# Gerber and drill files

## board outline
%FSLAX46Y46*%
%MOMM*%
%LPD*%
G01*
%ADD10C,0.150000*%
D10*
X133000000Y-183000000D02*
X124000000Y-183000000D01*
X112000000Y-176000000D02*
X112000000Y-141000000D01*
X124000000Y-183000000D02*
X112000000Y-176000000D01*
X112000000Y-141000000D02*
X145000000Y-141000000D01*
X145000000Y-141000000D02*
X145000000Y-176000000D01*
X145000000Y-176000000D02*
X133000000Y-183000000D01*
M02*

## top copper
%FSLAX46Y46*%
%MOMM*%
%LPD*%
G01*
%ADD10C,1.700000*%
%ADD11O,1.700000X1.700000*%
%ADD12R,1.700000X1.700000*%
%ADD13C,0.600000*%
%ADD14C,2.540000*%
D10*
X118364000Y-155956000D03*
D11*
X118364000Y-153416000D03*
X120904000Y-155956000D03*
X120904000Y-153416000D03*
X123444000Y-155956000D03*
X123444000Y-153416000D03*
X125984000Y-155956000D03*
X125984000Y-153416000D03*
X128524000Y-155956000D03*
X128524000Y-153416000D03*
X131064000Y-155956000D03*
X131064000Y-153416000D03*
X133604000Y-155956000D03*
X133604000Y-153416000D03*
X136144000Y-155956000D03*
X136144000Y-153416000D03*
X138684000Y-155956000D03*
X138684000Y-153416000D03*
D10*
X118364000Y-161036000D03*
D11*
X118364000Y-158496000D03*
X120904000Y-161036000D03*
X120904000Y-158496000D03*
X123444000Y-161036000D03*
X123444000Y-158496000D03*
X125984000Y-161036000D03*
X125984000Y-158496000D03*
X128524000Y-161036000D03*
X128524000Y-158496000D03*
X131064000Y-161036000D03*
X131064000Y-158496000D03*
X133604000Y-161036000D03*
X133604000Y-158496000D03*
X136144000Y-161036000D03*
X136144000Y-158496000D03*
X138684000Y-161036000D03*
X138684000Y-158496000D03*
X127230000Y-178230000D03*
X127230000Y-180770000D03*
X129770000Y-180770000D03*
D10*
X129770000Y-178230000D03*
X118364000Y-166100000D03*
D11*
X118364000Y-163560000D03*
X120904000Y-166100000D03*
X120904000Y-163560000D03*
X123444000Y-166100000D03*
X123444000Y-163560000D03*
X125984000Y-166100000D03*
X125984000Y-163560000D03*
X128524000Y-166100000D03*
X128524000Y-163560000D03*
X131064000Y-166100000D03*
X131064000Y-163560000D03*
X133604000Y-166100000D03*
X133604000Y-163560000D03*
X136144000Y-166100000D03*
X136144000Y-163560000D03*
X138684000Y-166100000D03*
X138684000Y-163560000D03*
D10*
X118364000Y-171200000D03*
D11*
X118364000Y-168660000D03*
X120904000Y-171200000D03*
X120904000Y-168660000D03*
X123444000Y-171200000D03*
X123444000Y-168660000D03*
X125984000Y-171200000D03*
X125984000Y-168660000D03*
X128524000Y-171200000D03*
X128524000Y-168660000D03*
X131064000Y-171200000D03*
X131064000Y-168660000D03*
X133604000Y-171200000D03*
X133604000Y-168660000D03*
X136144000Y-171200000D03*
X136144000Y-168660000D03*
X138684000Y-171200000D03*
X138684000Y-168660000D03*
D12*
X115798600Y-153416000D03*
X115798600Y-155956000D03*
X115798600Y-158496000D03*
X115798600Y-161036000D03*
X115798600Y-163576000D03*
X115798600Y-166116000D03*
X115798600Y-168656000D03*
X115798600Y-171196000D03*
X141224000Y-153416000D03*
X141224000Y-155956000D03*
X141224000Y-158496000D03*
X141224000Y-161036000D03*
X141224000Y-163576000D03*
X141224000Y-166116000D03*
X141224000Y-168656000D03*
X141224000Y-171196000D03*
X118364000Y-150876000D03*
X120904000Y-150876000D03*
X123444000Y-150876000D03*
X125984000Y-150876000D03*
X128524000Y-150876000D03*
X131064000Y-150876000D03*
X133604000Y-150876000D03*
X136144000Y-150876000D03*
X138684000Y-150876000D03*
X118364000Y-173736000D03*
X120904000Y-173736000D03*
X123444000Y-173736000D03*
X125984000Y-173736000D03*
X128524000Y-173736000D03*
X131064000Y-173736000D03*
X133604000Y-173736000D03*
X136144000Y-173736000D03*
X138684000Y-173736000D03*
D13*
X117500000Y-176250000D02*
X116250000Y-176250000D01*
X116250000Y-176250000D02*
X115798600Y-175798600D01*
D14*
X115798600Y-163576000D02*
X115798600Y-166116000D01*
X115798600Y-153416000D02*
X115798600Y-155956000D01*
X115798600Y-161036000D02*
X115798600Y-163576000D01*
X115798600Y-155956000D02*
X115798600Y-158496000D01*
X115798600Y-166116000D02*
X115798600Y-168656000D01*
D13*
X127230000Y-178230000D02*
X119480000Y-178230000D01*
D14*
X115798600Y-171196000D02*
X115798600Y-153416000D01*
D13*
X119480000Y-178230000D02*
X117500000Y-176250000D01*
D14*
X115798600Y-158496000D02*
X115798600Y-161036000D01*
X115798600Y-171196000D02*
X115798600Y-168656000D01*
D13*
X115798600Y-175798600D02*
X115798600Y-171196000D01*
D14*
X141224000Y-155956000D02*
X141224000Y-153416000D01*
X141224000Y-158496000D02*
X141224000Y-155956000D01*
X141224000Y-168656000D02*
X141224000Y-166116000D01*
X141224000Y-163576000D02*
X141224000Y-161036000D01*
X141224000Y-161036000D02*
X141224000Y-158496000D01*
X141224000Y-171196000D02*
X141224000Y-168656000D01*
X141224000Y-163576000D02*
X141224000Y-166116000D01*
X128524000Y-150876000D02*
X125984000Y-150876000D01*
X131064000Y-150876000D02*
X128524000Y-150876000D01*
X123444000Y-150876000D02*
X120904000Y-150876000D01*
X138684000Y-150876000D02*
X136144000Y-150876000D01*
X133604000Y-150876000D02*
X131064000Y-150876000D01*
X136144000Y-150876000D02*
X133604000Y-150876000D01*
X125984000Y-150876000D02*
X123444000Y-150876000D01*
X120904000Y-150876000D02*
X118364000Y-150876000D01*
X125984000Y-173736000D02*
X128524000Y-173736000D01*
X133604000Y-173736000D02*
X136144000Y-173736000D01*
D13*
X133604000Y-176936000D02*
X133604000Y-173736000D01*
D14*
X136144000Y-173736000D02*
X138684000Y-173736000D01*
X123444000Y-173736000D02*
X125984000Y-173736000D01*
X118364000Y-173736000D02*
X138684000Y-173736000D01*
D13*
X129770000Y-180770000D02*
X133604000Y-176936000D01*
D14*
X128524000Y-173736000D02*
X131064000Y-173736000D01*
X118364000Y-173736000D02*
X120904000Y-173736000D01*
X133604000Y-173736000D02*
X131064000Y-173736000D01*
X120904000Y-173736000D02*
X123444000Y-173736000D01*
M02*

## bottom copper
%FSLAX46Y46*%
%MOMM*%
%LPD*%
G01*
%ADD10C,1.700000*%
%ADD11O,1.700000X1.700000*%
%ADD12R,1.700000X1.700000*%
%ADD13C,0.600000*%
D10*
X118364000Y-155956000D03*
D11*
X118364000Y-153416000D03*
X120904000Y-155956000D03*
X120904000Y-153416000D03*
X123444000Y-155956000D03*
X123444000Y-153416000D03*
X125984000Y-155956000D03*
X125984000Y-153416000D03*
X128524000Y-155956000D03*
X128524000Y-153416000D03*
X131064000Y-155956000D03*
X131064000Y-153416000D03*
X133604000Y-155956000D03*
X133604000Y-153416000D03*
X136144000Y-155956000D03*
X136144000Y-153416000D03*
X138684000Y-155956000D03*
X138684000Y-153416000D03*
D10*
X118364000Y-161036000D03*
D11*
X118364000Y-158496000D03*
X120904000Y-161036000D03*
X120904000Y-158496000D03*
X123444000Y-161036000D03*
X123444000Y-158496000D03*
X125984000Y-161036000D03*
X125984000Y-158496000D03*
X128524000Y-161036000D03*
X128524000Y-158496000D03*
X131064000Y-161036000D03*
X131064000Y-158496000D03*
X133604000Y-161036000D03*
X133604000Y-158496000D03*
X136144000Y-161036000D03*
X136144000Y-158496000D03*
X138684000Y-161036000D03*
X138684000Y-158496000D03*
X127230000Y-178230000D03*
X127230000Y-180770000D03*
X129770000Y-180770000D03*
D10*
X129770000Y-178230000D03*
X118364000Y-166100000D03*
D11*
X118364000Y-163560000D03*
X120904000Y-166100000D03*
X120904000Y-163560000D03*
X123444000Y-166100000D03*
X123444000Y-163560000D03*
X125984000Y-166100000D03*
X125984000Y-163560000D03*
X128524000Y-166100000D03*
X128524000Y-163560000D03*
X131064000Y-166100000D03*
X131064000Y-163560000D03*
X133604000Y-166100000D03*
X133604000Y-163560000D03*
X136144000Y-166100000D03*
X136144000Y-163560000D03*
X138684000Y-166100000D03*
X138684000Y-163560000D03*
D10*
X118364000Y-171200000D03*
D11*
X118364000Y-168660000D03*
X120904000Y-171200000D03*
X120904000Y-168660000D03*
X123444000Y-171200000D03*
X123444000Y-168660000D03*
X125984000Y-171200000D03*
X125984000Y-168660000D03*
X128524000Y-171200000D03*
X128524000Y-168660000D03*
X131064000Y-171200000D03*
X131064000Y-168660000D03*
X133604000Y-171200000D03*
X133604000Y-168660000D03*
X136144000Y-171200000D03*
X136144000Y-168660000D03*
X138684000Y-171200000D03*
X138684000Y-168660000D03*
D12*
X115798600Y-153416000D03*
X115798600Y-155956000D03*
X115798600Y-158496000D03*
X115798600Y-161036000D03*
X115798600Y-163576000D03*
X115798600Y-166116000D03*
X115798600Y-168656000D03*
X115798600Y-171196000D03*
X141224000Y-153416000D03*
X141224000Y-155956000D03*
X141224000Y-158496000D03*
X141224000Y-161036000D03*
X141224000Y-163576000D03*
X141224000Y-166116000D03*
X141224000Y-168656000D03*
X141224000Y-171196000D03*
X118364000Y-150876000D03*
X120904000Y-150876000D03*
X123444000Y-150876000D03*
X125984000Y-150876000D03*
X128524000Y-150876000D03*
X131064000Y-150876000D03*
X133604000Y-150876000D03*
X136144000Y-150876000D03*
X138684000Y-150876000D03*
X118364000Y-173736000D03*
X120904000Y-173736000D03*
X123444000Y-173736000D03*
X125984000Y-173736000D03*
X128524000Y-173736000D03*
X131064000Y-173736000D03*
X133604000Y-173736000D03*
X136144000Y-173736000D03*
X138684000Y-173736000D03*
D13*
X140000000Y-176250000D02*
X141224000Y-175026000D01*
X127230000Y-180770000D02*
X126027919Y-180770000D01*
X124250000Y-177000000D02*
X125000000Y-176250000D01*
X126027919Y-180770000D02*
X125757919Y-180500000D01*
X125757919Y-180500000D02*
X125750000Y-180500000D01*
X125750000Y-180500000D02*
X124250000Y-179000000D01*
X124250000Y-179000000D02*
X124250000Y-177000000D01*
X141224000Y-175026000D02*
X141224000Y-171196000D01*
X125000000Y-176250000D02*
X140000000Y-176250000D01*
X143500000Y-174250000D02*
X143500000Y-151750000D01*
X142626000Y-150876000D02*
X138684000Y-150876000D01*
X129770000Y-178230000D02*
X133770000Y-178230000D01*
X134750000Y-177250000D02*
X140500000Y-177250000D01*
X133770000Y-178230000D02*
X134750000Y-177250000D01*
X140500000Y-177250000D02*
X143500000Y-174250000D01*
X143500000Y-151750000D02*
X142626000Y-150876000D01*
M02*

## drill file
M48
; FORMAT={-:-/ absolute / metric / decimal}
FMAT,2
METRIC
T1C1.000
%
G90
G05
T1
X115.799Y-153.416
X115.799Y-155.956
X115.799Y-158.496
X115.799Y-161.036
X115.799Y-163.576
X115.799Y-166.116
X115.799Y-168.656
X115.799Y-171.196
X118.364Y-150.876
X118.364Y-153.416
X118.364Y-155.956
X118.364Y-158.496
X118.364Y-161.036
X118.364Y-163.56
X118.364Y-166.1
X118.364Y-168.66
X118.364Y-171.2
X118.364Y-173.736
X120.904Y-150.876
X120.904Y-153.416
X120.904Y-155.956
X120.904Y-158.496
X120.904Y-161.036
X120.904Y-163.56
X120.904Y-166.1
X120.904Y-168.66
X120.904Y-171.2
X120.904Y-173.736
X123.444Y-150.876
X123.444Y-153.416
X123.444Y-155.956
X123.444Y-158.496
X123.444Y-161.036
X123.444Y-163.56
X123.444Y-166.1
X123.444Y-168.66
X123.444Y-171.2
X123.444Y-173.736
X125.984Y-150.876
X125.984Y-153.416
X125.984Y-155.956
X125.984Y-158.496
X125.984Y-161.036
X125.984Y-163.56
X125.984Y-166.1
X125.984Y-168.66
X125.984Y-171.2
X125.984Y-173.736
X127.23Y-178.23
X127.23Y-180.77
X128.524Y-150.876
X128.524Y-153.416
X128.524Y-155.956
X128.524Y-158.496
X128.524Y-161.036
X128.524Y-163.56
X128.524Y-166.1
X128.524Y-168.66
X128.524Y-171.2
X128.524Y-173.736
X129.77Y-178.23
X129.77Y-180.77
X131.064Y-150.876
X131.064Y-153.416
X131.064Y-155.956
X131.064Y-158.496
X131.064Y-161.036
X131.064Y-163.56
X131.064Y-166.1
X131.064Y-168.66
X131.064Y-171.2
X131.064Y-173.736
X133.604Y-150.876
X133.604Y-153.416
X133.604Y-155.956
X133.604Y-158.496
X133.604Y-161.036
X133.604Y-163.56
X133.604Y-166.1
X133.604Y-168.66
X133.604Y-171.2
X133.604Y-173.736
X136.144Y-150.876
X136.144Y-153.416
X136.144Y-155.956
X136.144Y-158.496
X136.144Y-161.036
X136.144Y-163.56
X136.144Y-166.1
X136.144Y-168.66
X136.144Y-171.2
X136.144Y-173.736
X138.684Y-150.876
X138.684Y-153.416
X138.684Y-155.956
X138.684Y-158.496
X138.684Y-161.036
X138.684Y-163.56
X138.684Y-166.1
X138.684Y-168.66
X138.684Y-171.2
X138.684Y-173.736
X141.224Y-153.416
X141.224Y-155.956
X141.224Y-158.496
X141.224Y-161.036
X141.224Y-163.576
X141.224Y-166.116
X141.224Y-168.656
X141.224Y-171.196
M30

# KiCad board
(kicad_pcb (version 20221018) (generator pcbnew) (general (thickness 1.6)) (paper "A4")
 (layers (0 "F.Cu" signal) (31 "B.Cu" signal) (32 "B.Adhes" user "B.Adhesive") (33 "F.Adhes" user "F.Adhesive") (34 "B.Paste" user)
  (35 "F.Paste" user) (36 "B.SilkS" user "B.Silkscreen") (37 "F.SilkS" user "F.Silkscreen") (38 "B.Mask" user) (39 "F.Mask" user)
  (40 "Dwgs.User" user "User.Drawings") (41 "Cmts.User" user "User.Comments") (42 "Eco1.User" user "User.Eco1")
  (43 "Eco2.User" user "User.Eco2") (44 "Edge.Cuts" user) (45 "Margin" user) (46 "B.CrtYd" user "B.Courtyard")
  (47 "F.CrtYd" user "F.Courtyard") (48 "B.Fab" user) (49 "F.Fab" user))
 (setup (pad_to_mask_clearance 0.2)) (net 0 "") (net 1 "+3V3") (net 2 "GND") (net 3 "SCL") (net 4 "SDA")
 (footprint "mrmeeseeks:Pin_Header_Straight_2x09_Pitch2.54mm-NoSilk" (layer "F.Cu") (at 118.364 155.956 90)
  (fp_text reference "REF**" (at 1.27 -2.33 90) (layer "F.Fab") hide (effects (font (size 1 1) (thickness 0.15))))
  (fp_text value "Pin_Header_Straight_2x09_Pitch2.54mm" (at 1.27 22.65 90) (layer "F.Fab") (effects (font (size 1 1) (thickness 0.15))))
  (pad "1" thru_hole circle (at 0 0 90) (size 1.7 1.7) (drill 1) (layers "*.Cu" "*.Mask"))
  (pad "2" thru_hole oval (at 2.54 0 90) (size 1.7 1.7) (drill 1) (layers "*.Cu" "*.Mask"))
  (pad "3" thru_hole oval (at 0 2.54 90) (size 1.7 1.7) (drill 1) (layers "*.Cu" "*.Mask"))
  (pad "4" thru_hole oval (at 2.54 2.54 90) (size 1.7 1.7) (drill 1) (layers "*.Cu" "*.Mask"))
  (pad "5" thru_hole oval (at 0 5.08 90) (size 1.7 1.7) (drill 1) (layers "*.Cu" "*.Mask"))
  (pad "6" thru_hole oval (at 2.54 5.08 90) (size 1.7 1.7) (drill 1) (layers "*.Cu" "*.Mask"))
  (pad "7" thru_hole oval (at 0 7.62 90) (size 1.7 1.7) (drill 1) (layers "*.Cu" "*.Mask"))
  (pad "8" thru_hole oval (at 2.54 7.62 90) (size 1.7 1.7) (drill 1) (layers "*.Cu" "*.Mask"))
  (pad "9" thru_hole oval (at 0 10.16 90) (size 1.7 1.7) (drill 1) (layers "*.Cu" "*.Mask"))
  (pad "10" thru_hole oval (at 2.54 10.16 90) (size 1.7 1.7) (drill 1) (layers "*.Cu" "*.Mask"))
  (pad "11" thru_hole oval (at 0 12.7 90) (size 1.7 1.7) (drill 1) (layers "*.Cu" "*.Mask"))
  (pad "12" thru_hole oval (at 2.54 12.7 90) (size 1.7 1.7) (drill 1) (layers "*.Cu" "*.Mask"))
  (pad "13" thru_hole oval (at 0 15.24 90) (size 1.7 1.7) (drill 1) (layers "*.Cu" "*.Mask"))
  (pad "14" thru_hole oval (at 2.54 15.24 90) (size 1.7 1.7) (drill 1) (layers "*.Cu" "*.Mask"))
  (pad "15" thru_hole oval (at 0 17.78 90) (size 1.7 1.7) (drill 1) (layers "*.Cu" "*.Mask"))
  (pad "16" thru_hole oval (at 2.54 17.78 90) (size 1.7 1.7) (drill 1) (layers "*.Cu" "*.Mask"))
  (pad "17" thru_hole oval (at 0 20.32 90) (size 1.7 1.7) (drill 1) (layers "*.Cu" "*.Mask"))
  (pad "18" thru_hole oval (at 2.54 20.32 90) (size 1.7 1.7) (drill 1) (layers "*.Cu" "*.Mask")))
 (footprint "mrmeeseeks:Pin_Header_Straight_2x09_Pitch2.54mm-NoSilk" (layer "F.Cu") (at 118.364 161.036 90)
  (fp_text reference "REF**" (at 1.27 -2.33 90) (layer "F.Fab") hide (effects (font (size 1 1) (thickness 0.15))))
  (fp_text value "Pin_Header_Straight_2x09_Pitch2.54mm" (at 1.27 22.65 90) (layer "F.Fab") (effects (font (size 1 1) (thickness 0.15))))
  (pad "1" thru_hole circle (at 0 0 90) (size 1.7 1.7) (drill 1) (layers "*.Cu" "*.Mask"))
  (pad "2" thru_hole oval (at 2.54 0 90) (size 1.7 1.7) (drill 1) (layers "*.Cu" "*.Mask"))
  (pad "3" thru_hole oval (at 0 2.54 90) (size 1.7 1.7) (drill 1) (layers "*.Cu" "*.Mask"))
  (pad "4" thru_hole oval (at 2.54 2.54 90) (size 1.7 1.7) (drill 1) (layers "*.Cu" "*.Mask"))
  (pad "5" thru_hole oval (at 0 5.08 90) (size 1.7 1.7) (drill 1) (layers "*.Cu" "*.Mask"))
  (pad "6" thru_hole oval (at 2.54 5.08 90) (size 1.7 1.7) (drill 1) (layers "*.Cu" "*.Mask"))
  (pad "7" thru_hole oval (at 0 7.62 90) (size 1.7 1.7) (drill 1) (layers "*.Cu" "*.Mask"))
  (pad "8" thru_hole oval (at 2.54 7.62 90) (size 1.7 1.7) (drill 1) (layers "*.Cu" "*.Mask"))
  (pad "9" thru_hole oval (at 0 10.16 90) (size 1.7 1.7) (drill 1) (layers "*.Cu" "*.Mask"))
  (pad "10" thru_hole oval (at 2.54 10.16 90) (size 1.7 1.7) (drill 1) (layers "*.Cu" "*.Mask"))
  (pad "11" thru_hole oval (at 0 12.7 90) (size 1.7 1.7) (drill 1) (layers "*.Cu" "*.Mask"))
  (pad "12" thru_hole oval (at 2.54 12.7 90) (size 1.7 1.7) (drill 1) (layers "*.Cu" "*.Mask"))
  (pad "13" thru_hole oval (at 0 15.24 90) (size 1.7 1.7) (drill 1) (layers "*.Cu" "*.Mask"))
  (pad "14" thru_hole oval (at 2.54 15.24 90) (size 1.7 1.7) (drill 1) (layers "*.Cu" "*.Mask"))
  (pad "15" thru_hole oval (at 0 17.78 90) (size 1.7 1.7) (drill 1) (layers "*.Cu" "*.Mask"))
  (pad "16" thru_hole oval (at 2.54 17.78 90) (size 1.7 1.7) (drill 1) (layers "*.Cu" "*.Mask"))
  (pad "17" thru_hole oval (at 0 20.32 90) (size 1.7 1.7) (drill 1) (layers "*.Cu" "*.Mask"))
  (pad "18" thru_hole oval (at 2.54 20.32 90) (size 1.7 1.7) (drill 1) (layers "*.Cu" "*.Mask")))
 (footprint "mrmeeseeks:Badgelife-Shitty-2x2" (layer "F.Cu") (at 128.5 179.5)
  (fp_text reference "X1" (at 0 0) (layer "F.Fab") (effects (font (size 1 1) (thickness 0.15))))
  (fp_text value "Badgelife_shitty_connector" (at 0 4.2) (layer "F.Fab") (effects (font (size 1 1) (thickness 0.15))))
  (pad "1" thru_hole oval (at -1.27 -1.27) (size 1.7 1.7) (drill 1) (layers "*.Cu" "*.Mask") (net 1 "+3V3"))
  (pad "2" thru_hole oval (at -1.27 1.27) (size 1.7 1.7) (drill 1) (layers "*.Cu" "*.Mask") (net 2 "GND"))
  (pad "3" thru_hole oval (at 1.27 1.27) (size 1.7 1.7) (drill 1) (layers "*.Cu" "*.Mask") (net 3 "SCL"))
  (pad "4" thru_hole circle (at 1.27 -1.27) (size 1.7 1.7) (drill 1) (layers "*.Cu" "*.Mask") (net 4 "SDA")))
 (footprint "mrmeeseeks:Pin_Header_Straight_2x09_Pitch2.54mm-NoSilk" (layer "F.Cu") (at 118.364 166.1 90)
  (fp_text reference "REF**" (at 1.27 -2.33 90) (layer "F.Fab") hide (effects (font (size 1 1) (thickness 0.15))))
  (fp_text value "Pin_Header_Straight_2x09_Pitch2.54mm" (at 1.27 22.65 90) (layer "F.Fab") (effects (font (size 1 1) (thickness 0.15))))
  (pad "1" thru_hole circle (at 0 0 90) (size 1.7 1.7) (drill 1) (layers "*.Cu" "*.Mask"))
  (pad "2" thru_hole oval (at 2.54 0 90) (size 1.7 1.7) (drill 1) (layers "*.Cu" "*.Mask"))
  (pad "3" thru_hole oval (at 0 2.54 90) (size 1.7 1.7) (drill 1) (layers "*.Cu" "*.Mask"))
  (pad "4" thru_hole oval (at 2.54 2.54 90) (size 1.7 1.7) (drill 1) (layers "*.Cu" "*.Mask"))
  (pad "5" thru_hole oval (at 0 5.08 90) (size 1.7 1.7) (drill 1) (layers "*.Cu" "*.Mask"))
  (pad "6" thru_hole oval (at 2.54 5.08 90) (size 1.7 1.7) (drill 1) (layers "*.Cu" "*.Mask"))
  (pad "7" thru_hole oval (at 0 7.62 90) (size 1.7 1.7) (drill 1) (layers "*.Cu" "*.Mask"))
  (pad "8" thru_hole oval (at 2.54 7.62 90) (size 1.7 1.7) (drill 1) (layers "*.Cu" "*.Mask"))
  (pad "9" thru_hole oval (at 0 10.16 90) (size 1.7 1.7) (drill 1) (layers "*.Cu" "*.Mask"))
  (pad "10" thru_hole oval (at 2.54 10.16 90) (size 1.7 1.7) (drill 1) (layers "*.Cu" "*.Mask"))
  (pad "11" thru_hole oval (at 0 12.7 90) (size 1.7 1.7) (drill 1) (layers "*.Cu" "*.Mask"))
  (pad "12" thru_hole oval (at 2.54 12.7 90) (size 1.7 1.7) (drill 1) (layers "*.Cu" "*.Mask"))
  (pad "13" thru_hole oval (at 0 15.24 90) (size 1.7 1.7) (drill 1) (layers "*.Cu" "*.Mask"))
  (pad "14" thru_hole oval (at 2.54 15.24 90) (size 1.7 1.7) (drill 1) (layers "*.Cu" "*.Mask"))
  (pad "15" thru_hole oval (at 0 17.78 90) (size 1.7 1.7) (drill 1) (layers "*.Cu" "*.Mask"))
  (pad "16" thru_hole oval (at 2.54 17.78 90) (size 1.7 1.7) (drill 1) (layers "*.Cu" "*.Mask"))
  (pad "17" thru_hole oval (at 0 20.32 90) (size 1.7 1.7) (drill 1) (layers "*.Cu" "*.Mask"))
  (pad "18" thru_hole oval (at 2.54 20.32 90) (size 1.7 1.7) (drill 1) (layers "*.Cu" "*.Mask")))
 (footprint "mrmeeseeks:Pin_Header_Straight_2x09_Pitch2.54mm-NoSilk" (layer "F.Cu") (at 118.364 171.2 90)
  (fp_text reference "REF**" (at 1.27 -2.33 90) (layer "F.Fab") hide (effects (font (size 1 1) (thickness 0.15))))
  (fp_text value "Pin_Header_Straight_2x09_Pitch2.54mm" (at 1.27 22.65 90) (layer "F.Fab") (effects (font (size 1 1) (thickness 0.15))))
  (pad "1" thru_hole circle (at 0 0 90) (size 1.7 1.7) (drill 1) (layers "*.Cu" "*.Mask"))
  (pad "2" thru_hole oval (at 2.54 0 90) (size 1.7 1.7) (drill 1) (layers "*.Cu" "*.Mask"))
  (pad "3" thru_hole oval (at 0 2.54 90) (size 1.7 1.7) (drill 1) (layers "*.Cu" "*.Mask"))
  (pad "4" thru_hole oval (at 2.54 2.54 90) (size 1.7 1.7) (drill 1) (layers "*.Cu" "*.Mask"))
  (pad "5" thru_hole oval (at 0 5.08 90) (size 1.7 1.7) (drill 1) (layers "*.Cu" "*.Mask"))
  (pad "6" thru_hole oval (at 2.54 5.08 90) (size 1.7 1.7) (drill 1) (layers "*.Cu" "*.Mask"))
  (pad "7" thru_hole oval (at 0 7.62 90) (size 1.7 1.7) (drill 1) (layers "*.Cu" "*.Mask"))
  (pad "8" thru_hole oval (at 2.54 7.62 90) (size 1.7 1.7) (drill 1) (layers "*.Cu" "*.Mask"))
  (pad "9" thru_hole oval (at 0 10.16 90) (size 1.7 1.7) (drill 1) (layers "*.Cu" "*.Mask"))
  (pad "10" thru_hole oval (at 2.54 10.16 90) (size 1.7 1.7) (drill 1) (layers "*.Cu" "*.Mask"))
  (pad "11" thru_hole oval (at 0 12.7 90) (size 1.7 1.7) (drill 1) (layers "*.Cu" "*.Mask"))
  (pad "12" thru_hole oval (at 2.54 12.7 90) (size 1.7 1.7) (drill 1) (layers "*.Cu" "*.Mask"))
  (pad "13" thru_hole oval (at 0 15.24 90) (size 1.7 1.7) (drill 1) (layers "*.Cu" "*.Mask"))
  (pad "14" thru_hole oval (at 2.54 15.24 90) (size 1.7 1.7) (drill 1) (layers "*.Cu" "*.Mask"))
  (pad "15" thru_hole oval (at 0 17.78 90) (size 1.7 1.7) (drill 1) (layers "*.Cu" "*.Mask"))
  (pad "16" thru_hole oval (at 2.54 17.78 90) (size 1.7 1.7) (drill 1) (layers "*.Cu" "*.Mask"))
  (pad "17" thru_hole oval (at 0 20.32 90) (size 1.7 1.7) (drill 1) (layers "*.Cu" "*.Mask"))
  (pad "18" thru_hole oval (at 2.54 20.32 90) (size 1.7 1.7) (drill 1) (layers "*.Cu" "*.Mask")))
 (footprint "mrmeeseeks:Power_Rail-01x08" (layer "F.Cu") (at 115.7986 153.416)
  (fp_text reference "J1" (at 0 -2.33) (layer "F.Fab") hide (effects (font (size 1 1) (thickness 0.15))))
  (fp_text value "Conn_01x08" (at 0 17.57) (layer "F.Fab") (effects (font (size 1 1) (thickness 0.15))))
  (pad "1" thru_hole rect (at 0 0) (size 1.7 1.7) (drill 1) (layers "*.Cu" "*.Mask") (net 1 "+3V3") (solder_mask_margin 0.1))
  (pad "2" thru_hole rect (at 0 2.54) (size 1.7 1.7) (drill 1) (layers "*.Cu" "*.Mask") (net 1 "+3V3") (solder_mask_margin 0.1))
  (pad "3" thru_hole rect (at 0 5.08) (size 1.7 1.7) (drill 1) (layers "*.Cu" "*.Mask") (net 1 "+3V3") (solder_mask_margin 0.1))
  (pad "4" thru_hole rect (at 0 7.62) (size 1.7 1.7) (drill 1) (layers "*.Cu" "*.Mask") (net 1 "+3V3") (solder_mask_margin 0.1))
  (pad "5" thru_hole rect (at 0 10.16) (size 1.7 1.7) (drill 1) (layers "*.Cu" "*.Mask") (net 1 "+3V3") (solder_mask_margin 0.1))
  (pad "6" thru_hole rect (at 0 12.7) (size 1.7 1.7) (drill 1) (layers "*.Cu" "*.Mask") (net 1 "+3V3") (solder_mask_margin 0.1))
  (pad "7" thru_hole rect (at 0 15.24) (size 1.7 1.7) (drill 1) (layers "*.Cu" "*.Mask") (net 1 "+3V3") (solder_mask_margin 0.1))
  (pad "8" thru_hole rect (at 0 17.78) (size 1.7 1.7) (drill 1) (layers "*.Cu" "*.Mask") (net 1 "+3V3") (solder_mask_margin 0.1)))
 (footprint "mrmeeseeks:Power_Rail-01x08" (layer "F.Cu") (at 141.224 153.416)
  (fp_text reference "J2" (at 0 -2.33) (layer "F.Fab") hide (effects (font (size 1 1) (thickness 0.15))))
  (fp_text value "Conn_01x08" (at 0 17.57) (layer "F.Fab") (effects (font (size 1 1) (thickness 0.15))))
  (pad "1" thru_hole rect (at 0 0) (size 1.7 1.7) (drill 1) (layers "*.Cu" "*.Mask") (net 2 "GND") (solder_mask_margin 0.1))
  (pad "2" thru_hole rect (at 0 2.54) (size 1.7 1.7) (drill 1) (layers "*.Cu" "*.Mask") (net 2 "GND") (solder_mask_margin 0.1))
  (pad "3" thru_hole rect (at 0 5.08) (size 1.7 1.7) (drill 1) (layers "*.Cu" "*.Mask") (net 2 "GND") (solder_mask_margin 0.1))
  (pad "4" thru_hole rect (at 0 7.62) (size 1.7 1.7) (drill 1) (layers "*.Cu" "*.Mask") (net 2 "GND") (solder_mask_margin 0.1))
  (pad "5" thru_hole rect (at 0 10.16) (size 1.7 1.7) (drill 1) (layers "*.Cu" "*.Mask") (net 2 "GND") (solder_mask_margin 0.1))
  (pad "6" thru_hole rect (at 0 12.7) (size 1.7 1.7) (drill 1) (layers "*.Cu" "*.Mask") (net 2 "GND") (solder_mask_margin 0.1))
  (pad "7" thru_hole rect (at 0 15.24) (size 1.7 1.7) (drill 1) (layers "*.Cu" "*.Mask") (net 2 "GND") (solder_mask_margin 0.1))
  (pad "8" thru_hole rect (at 0 17.78) (size 1.7 1.7) (drill 1) (layers "*.Cu" "*.Mask") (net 2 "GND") (solder_mask_margin 0.1)))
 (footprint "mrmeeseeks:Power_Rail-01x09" (layer "F.Cu") (at 118.364 150.876 90)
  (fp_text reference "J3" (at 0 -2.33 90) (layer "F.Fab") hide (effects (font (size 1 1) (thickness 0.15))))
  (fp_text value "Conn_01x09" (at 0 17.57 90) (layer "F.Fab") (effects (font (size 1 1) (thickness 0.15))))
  (pad "1" thru_hole rect (at 0 0 90) (size 1.7 1.7) (drill 1) (layers "*.Cu" "*.Mask") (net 4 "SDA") (solder_mask_margin 0.1))
  (pad "2" thru_hole rect (at 0 2.54 90) (size 1.7 1.7) (drill 1) (layers "*.Cu" "*.Mask") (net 4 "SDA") (solder_mask_margin 0.1))
  (pad "3" thru_hole rect (at 0 5.08 90) (size 1.7 1.7) (drill 1) (layers "*.Cu" "*.Mask") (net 4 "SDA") (solder_mask_margin 0.1))
  (pad "4" thru_hole rect (at 0 7.62 90) (size 1.7 1.7) (drill 1) (layers "*.Cu" "*.Mask") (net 4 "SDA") (solder_mask_margin 0.1))
  (pad "5" thru_hole rect (at 0 10.16 90) (size 1.7 1.7) (drill 1) (layers "*.Cu" "*.Mask") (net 4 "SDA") (solder_mask_margin 0.1))
  (pad "6" thru_hole rect (at 0 12.7 90) (size 1.7 1.7) (drill 1) (layers "*.Cu" "*.Mask") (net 4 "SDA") (solder_mask_margin 0.1))
  (pad "7" thru_hole rect (at 0 15.24 90) (size 1.7 1.7) (drill 1) (layers "*.Cu" "*.Mask") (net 4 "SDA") (solder_mask_margin 0.1))
  (pad "8" thru_hole rect (at 0 17.78 90) (size 1.7 1.7) (drill 1) (layers "*.Cu" "*.Mask") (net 4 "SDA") (solder_mask_margin 0.1))
  (pad "9" thru_hole rect (at 0 20.32 90) (size 1.7 1.7) (drill 1) (layers "*.Cu" "*.Mask") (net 4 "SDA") (solder_mask_margin 0.1)))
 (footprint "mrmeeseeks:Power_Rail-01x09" (layer "F.Cu") (at 118.364 173.736 90)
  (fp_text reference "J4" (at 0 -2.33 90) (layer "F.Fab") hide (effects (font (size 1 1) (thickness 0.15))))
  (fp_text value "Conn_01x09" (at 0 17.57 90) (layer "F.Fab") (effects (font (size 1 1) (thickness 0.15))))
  (pad "1" thru_hole rect (at 0 0 90) (size 1.7 1.7) (drill 1) (layers "*.Cu" "*.Mask") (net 3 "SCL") (solder_mask_margin 0.1))
  (pad "2" thru_hole rect (at 0 2.54 90) (size 1.7 1.7) (drill 1) (layers "*.Cu" "*.Mask") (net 3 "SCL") (solder_mask_margin 0.1))
  (pad "3" thru_hole rect (at 0 5.08 90) (size 1.7 1.7) (drill 1) (layers "*.Cu" "*.Mask") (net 3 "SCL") (solder_mask_margin 0.1))
  (pad "4" thru_hole rect (at 0 7.62 90) (size 1.7 1.7) (drill 1) (layers "*.Cu" "*.Mask") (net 3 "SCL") (solder_mask_margin 0.1))
  (pad "5" thru_hole rect (at 0 10.16 90) (size 1.7 1.7) (drill 1) (layers "*.Cu" "*.Mask") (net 3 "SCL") (solder_mask_margin 0.1))
  (pad "6" thru_hole rect (at 0 12.7 90) (size 1.7 1.7) (drill 1) (layers "*.Cu" "*.Mask") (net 3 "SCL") (solder_mask_margin 0.1))
  (pad "7" thru_hole rect (at 0 15.24 90) (size 1.7 1.7) (drill 1) (layers "*.Cu" "*.Mask") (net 3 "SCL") (solder_mask_margin 0.1))
  (pad "8" thru_hole rect (at 0 17.78 90) (size 1.7 1.7) (drill 1) (layers "*.Cu" "*.Mask") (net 3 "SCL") (solder_mask_margin 0.1))
  (pad "9" thru_hole rect (at 0 20.32 90) (size 1.7 1.7) (drill 1) (layers "*.Cu" "*.Mask") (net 3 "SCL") (solder_mask_margin 0.1)))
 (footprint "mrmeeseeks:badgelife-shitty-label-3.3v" (layer "F.Cu") (at 113.4 162.2 90)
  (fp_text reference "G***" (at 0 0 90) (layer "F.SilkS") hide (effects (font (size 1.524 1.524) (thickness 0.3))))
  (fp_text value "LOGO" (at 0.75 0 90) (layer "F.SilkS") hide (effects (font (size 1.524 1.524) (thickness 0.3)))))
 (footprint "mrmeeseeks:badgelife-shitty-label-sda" (layer "F.Cu") (at 128.2 148.8)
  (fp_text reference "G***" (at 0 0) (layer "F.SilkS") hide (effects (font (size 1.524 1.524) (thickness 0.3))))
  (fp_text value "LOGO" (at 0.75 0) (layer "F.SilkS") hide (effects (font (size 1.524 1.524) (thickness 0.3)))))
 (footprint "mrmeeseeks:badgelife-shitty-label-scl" (layer "F.Cu") (at 128.4 175.7)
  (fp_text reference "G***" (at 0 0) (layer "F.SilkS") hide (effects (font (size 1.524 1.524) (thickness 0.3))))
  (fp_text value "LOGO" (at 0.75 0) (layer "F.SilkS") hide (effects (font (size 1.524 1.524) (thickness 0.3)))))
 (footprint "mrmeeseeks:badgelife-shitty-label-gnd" (layer "F.Cu") (at 143.7 162.3 -90)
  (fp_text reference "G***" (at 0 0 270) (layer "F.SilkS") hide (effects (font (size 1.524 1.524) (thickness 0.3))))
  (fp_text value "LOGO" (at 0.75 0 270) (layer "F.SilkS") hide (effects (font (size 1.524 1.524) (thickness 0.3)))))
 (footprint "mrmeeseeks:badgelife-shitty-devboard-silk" (layer "F.Cu") (at 128.9 144.6)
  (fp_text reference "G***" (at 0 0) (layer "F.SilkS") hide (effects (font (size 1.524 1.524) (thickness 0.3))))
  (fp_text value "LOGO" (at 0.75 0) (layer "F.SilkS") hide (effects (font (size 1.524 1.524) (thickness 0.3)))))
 (gr_line (start 133 183) (end 124 183) (stroke (width 0.15) (type solid)) (layer "Edge.Cuts"))
 (gr_line (start 112 176) (end 112 141) (stroke (width 0.15) (type solid)) (layer "Edge.Cuts"))
 (gr_line (start 124 183) (end 112 176) (stroke (width 0.15) (type solid)) (layer "Edge.Cuts"))
 (gr_line (start 112 141) (end 145 141) (stroke (width 0.15) (type solid)) (layer "Edge.Cuts"))
 (gr_line (start 145 141) (end 145 176) (stroke (width 0.15) (type solid)) (layer "Edge.Cuts"))
 (gr_line (start 145 176) (end 133 183) (stroke (width 0.15) (type solid)) (layer "Edge.Cuts"))
 (segment (start 117.5 176.25) (end 116.25 176.25) (width 0.6) (layer "F.Cu") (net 1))
 (segment (start 116.25 176.25) (end 115.7986 175.7986) (width 0.6) (layer "F.Cu") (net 1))
 (segment (start 115.7986 163.576) (end 115.7986 166.116) (width 2.54) (layer "F.Cu") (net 1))
 (segment (start 115.7986 153.416) (end 115.7986 155.956) (width 2.54) (layer "F.Cu") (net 1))
 (segment (start 115.7986 161.036) (end 115.7986 163.576) (width 2.54) (layer "F.Cu") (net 1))
 (segment (start 115.7986 155.956) (end 115.7986 158.496) (width 2.54) (layer "F.Cu") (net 1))
 (segment (start 115.7986 166.116) (end 115.7986 168.656) (width 2.54) (layer "F.Cu") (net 1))
 (segment (start 127.23 178.23) (end 119.48 178.23) (width 0.6) (layer "F.Cu") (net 1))
 (segment (start 115.7986 171.196) (end 115.7986 153.416) (width 2.54) (layer "F.Cu") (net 1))
 (segment (start 119.48 178.23) (end 117.5 176.25) (width 0.6) (layer "F.Cu") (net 1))
 (segment (start 115.7986 158.496) (end 115.7986 161.036) (width 2.54) (layer "F.Cu") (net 1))
 (segment (start 115.7986 171.196) (end 115.7986 168.656) (width 2.54) (layer "F.Cu") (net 1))
 (segment (start 115.7986 175.7986) (end 115.7986 171.196) (width 0.6) (layer "F.Cu") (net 1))
 (segment (start 141.224 155.956) (end 141.224 153.416) (width 2.54) (layer "F.Cu") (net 2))
 (segment (start 141.224 158.496) (end 141.224 155.956) (width 2.54) (layer "F.Cu") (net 2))
 (segment (start 141.224 168.656) (end 141.224 166.116) (width 2.54) (layer "F.Cu") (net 2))
 (segment (start 141.224 163.576) (end 141.224 161.036) (width 2.54) (layer "F.Cu") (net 2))
 (segment (start 141.224 161.036) (end 141.224 158.496) (width 2.54) (layer "F.Cu") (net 2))
 (segment (start 141.224 171.196) (end 141.224 168.656) (width 2.54) (layer "F.Cu") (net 2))
 (segment (start 141.224 163.576) (end 141.224 166.116) (width 2.54) (layer "F.Cu") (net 2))
 (segment (start 140 176.25) (end 141.224 175.026) (width 0.6) (layer "B.Cu") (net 2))
 (segment (start 127.23 180.77) (end 126.027919 180.77) (width 0.6) (layer "B.Cu") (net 2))
 (segment (start 124.25 177) (end 125 176.25) (width 0.6) (layer "B.Cu") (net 2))
 (segment (start 126.027919 180.77) (end 125.757919 180.5) (width 0.6) (layer "B.Cu") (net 2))
 (segment (start 125.757919 180.5) (end 125.75 180.5) (width 0.6) (layer "B.Cu") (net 2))
 (segment (start 125.75 180.5) (end 124.25 179) (width 0.6) (layer "B.Cu") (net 2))
 (segment (start 124.25 179) (end 124.25 177) (width 0.6) (layer "B.Cu") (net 2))
 (segment (start 141.224 175.026) (end 141.224 171.196) (width 0.6) (layer "B.Cu") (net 2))
 (segment (start 125 176.25) (end 140 176.25) (width 0.6) (layer "B.Cu") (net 2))
 (segment (start 128.524 150.876) (end 125.984 150.876) (width 2.54) (layer "F.Cu") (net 4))
 (segment (start 131.064 150.876) (end 128.524 150.876) (width 2.54) (layer "F.Cu") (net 4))
 (segment (start 123.444 150.876) (end 120.904 150.876) (width 2.54) (layer "F.Cu") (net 4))
 (segment (start 138.684 150.876) (end 136.144 150.876) (width 2.54) (layer "F.Cu") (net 4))
 (segment (start 133.604 150.876) (end 131.064 150.876) (width 2.54) (layer "F.Cu") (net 4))
 (segment (start 136.144 150.876) (end 133.604 150.876) (width 2.54) (layer "F.Cu") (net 4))
 (segment (start 125.984 150.876) (end 123.444 150.876) (width 2.54) (layer "F.Cu") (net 4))
 (segment (start 120.904 150.876) (end 118.364 150.876) (width 2.54) (layer "F.Cu") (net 4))
 (segment (start 143.5 174.25) (end 143.5 151.75) (width 0.6) (layer "B.Cu") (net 4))
 (segment (start 142.626 150.876) (end 138.684 150.876) (width 0.6) (layer "B.Cu") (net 4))
 (segment (start 129.77 178.23) (end 133.77 178.23) (width 0.6) (layer "B.Cu") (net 4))
 (segment (start 134.75 177.25) (end 140.5 177.25) (width 0.6) (layer "B.Cu") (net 4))
 (segment (start 133.77 178.23) (end 134.75 177.25) (width 0.6) (layer "B.Cu") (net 4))
 (segment (start 140.5 177.25) (end 143.5 174.25) (width 0.6) (layer "B.Cu") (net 4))
 (segment (start 143.5 151.75) (end 142.626 150.876) (width 0.6) (layer "B.Cu") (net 4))
 (segment (start 125.984 173.736) (end 128.524 173.736) (width 2.54) (layer "F.Cu") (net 3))
 (segment (start 133.604 173.736) (end 136.144 173.736) (width 2.54) (layer "F.Cu") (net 3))
 (segment (start 133.604 176.936) (end 133.604 173.736) (width 0.6) (layer "F.Cu") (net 3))
 (segment (start 136.144 173.736) (end 138.684 173.736) (width 2.54) (layer "F.Cu") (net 3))
 (segment (start 123.444 173.736) (end 125.984 173.736) (width 2.54) (layer "F.Cu") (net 3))
 (segment (start 118.364 173.736) (end 138.684 173.736) (width 2.54) (layer "F.Cu") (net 3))
 (segment (start 129.77 180.77) (end 133.604 176.936) (width 0.6) (layer "F.Cu") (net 3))
 (segment (start 128.524 173.736) (end 131.064 173.736) (width 2.54) (layer "F.Cu") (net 3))
 (segment (start 118.364 173.736) (end 120.904 173.736) (width 2.54) (layer "F.Cu") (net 3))
 (segment (start 133.604 173.736) (end 131.064 173.736) (width 2.54) (layer "F.Cu") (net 3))
 (segment (start 120.904 173.736) (end 123.444 173.736) (width 2.54) (layer "F.Cu") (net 3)))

